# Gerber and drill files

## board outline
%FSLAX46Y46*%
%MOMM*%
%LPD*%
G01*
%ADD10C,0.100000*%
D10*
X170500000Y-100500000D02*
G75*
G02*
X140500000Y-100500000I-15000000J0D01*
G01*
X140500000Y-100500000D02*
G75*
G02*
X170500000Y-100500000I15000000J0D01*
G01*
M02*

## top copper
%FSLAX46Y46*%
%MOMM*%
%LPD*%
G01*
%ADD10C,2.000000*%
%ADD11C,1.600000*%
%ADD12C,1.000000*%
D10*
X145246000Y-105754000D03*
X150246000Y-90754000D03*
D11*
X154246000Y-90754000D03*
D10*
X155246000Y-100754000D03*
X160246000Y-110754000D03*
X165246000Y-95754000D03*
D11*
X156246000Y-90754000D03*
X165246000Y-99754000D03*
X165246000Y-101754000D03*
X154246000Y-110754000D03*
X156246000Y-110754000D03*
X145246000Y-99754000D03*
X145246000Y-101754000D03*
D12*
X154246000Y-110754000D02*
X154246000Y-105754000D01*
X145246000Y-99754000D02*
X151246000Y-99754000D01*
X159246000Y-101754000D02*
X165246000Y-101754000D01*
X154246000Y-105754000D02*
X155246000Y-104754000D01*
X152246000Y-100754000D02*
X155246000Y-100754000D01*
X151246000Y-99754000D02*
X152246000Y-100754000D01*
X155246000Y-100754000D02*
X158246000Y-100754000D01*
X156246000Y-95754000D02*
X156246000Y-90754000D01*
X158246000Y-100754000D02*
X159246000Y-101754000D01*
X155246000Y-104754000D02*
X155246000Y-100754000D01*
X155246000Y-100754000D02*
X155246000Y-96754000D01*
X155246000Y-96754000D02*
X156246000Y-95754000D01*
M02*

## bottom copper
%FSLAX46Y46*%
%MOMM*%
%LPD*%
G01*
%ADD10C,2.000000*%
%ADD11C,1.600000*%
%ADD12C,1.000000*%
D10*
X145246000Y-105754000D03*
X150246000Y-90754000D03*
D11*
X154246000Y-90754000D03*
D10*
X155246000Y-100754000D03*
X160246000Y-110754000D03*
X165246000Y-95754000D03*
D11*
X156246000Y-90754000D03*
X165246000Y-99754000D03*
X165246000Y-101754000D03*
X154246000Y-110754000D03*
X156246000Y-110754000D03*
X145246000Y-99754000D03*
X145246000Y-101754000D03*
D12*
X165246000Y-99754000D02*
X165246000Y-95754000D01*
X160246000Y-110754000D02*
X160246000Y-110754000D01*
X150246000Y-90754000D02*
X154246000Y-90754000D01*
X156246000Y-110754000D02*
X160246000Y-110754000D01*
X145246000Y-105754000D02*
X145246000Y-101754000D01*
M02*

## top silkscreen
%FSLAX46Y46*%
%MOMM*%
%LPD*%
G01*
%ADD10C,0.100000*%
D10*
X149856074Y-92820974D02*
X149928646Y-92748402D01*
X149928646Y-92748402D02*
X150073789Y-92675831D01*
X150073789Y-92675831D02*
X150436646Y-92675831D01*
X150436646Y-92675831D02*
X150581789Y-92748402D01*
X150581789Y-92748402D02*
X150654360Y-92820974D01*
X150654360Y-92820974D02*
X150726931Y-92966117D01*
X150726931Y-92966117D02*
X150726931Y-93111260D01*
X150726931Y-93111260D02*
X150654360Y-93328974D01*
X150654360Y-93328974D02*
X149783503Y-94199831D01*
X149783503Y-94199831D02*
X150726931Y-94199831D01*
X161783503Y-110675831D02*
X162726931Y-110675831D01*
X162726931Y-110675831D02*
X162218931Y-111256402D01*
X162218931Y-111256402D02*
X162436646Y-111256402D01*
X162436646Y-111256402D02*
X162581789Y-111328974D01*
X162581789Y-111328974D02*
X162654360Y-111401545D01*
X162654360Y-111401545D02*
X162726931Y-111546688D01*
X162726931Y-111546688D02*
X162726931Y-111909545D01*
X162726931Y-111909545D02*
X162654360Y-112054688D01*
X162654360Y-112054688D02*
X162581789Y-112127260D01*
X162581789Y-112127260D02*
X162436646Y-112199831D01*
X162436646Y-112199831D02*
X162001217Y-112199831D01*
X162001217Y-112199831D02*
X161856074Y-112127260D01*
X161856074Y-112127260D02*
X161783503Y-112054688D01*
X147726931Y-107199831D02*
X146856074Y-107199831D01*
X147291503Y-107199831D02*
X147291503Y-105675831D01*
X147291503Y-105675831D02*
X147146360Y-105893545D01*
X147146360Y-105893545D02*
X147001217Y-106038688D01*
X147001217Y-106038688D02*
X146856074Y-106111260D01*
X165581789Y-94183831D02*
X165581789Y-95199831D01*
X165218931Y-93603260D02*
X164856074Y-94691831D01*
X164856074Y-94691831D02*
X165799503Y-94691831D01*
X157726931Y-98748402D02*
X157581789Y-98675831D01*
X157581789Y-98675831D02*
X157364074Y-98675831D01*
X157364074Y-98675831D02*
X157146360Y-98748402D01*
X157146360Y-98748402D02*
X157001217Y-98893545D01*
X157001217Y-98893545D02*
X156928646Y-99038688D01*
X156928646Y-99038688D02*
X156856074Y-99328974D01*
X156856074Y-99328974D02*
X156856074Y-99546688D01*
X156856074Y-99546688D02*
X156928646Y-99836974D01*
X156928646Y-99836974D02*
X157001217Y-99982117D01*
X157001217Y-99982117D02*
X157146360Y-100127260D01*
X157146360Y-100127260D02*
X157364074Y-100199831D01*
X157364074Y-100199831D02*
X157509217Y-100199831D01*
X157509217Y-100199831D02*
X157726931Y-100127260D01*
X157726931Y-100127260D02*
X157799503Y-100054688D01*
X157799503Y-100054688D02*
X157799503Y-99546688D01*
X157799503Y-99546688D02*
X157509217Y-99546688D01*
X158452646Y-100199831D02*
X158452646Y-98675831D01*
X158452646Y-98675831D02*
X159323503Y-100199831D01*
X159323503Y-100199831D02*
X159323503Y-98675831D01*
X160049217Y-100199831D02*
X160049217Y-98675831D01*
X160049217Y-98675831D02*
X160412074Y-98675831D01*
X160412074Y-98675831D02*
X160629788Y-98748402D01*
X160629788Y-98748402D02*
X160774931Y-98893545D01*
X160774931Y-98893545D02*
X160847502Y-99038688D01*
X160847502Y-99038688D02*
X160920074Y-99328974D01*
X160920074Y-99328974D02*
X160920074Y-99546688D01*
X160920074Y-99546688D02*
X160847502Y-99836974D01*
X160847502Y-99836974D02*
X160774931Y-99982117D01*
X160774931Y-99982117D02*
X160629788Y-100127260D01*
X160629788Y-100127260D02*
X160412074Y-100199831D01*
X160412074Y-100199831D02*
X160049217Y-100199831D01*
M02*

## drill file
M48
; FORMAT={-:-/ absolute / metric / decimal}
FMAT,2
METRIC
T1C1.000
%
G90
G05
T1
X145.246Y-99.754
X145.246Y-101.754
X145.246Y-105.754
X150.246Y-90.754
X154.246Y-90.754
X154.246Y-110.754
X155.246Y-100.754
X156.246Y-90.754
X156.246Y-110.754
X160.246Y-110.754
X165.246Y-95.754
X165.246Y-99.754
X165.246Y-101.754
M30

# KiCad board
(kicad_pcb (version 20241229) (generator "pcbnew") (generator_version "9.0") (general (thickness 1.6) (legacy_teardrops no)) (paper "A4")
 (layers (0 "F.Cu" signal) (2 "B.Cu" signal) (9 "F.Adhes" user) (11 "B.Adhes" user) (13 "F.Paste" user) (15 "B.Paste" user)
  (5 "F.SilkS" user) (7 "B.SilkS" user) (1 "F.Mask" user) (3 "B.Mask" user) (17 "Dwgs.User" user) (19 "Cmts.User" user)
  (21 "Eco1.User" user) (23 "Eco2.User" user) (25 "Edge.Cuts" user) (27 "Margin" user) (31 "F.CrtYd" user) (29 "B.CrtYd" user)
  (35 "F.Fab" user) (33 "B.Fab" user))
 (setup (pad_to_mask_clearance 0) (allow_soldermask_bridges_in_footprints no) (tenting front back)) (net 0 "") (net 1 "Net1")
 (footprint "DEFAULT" (layer "F.Cu") (at 61.246 195.754)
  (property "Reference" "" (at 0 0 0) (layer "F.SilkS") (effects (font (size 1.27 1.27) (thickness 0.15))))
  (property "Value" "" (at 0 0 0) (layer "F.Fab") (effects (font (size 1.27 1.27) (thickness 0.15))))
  (pad "173" thru_hole circle (at 84 -90) (size 2 2) (drill 1) (layers "*.Cu") (remove_unused_layers no))
  (pad "173" thru_hole circle (at 89 -105) (size 2 2) (drill 1) (layers "*.Cu") (remove_unused_layers no))
  (pad "173" thru_hole circle (at 93 -105) (size 1.6 1.6) (drill 1) (layers "*.Cu") (remove_unused_layers no))
  (pad "173" thru_hole circle (at 94 -95) (size 2 2) (drill 1) (layers "*.Cu") (remove_unused_layers no))
  (pad "173" thru_hole circle (at 99 -85) (size 2 2) (drill 1) (layers "*.Cu") (remove_unused_layers no))
  (pad "173" thru_hole circle (at 104 -100) (size 2 2) (drill 1) (layers "*.Cu") (remove_unused_layers no))
  (pad "174" thru_hole circle (at 95 -105) (size 1.6 1.6) (drill 1) (layers "*.Cu") (remove_unused_layers no))
  (pad "175" thru_hole circle (at 104 -96) (size 1.6 1.6) (drill 1) (layers "*.Cu") (remove_unused_layers no))
  (pad "176" thru_hole circle (at 104 -94) (size 1.6 1.6) (drill 1) (layers "*.Cu") (remove_unused_layers no))
  (pad "177" thru_hole circle (at 93 -85) (size 1.6 1.6) (drill 1) (layers "*.Cu") (remove_unused_layers no))
  (pad "178" thru_hole circle (at 95 -85) (size 1.6 1.6) (drill 1) (layers "*.Cu") (remove_unused_layers no))
  (pad "179" thru_hole circle (at 84 -96) (size 1.6 1.6) (drill 1) (layers "*.Cu") (remove_unused_layers no))
  (pad "180" thru_hole circle (at 84 -94) (size 1.6 1.6) (drill 1) (layers "*.Cu") (remove_unused_layers no)))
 (gr_circle (center 155.5 100.5) (end 170.5 100.5) (stroke (width 0.1) (type solid)) (fill no) (layer "Edge.Cuts"))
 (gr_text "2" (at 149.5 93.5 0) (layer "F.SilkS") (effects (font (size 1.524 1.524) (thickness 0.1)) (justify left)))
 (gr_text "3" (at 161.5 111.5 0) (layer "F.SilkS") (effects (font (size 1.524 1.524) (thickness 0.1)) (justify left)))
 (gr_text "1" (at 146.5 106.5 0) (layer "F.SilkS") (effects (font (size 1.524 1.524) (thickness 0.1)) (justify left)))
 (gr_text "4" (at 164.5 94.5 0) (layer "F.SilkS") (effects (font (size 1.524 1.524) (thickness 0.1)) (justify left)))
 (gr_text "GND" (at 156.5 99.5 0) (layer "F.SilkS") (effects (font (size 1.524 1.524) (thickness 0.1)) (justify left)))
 (segment (start 154.246 110.754) (end 154.246 105.754) (width 1) (layer "F.Cu") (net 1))
 (segment (start 145.246 99.754) (end 151.246 99.754) (width 1) (layer "F.Cu") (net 1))
 (segment (start 159.246 101.754) (end 165.246 101.754) (width 1) (layer "F.Cu") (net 1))
 (segment (start 154.246 105.754) (end 155.246 104.754) (width 1) (layer "F.Cu") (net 1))
 (segment (start 152.246 100.754) (end 155.246 100.754) (width 1) (layer "F.Cu") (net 1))
 (segment (start 151.246 99.754) (end 152.246 100.754) (width 1) (layer "F.Cu") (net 1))
 (segment (start 155.246 100.754) (end 158.246 100.754) (width 1) (layer "F.Cu") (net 1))
 (segment (start 156.246 95.754) (end 156.246 90.754) (width 1) (layer "F.Cu") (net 1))
 (segment (start 158.246 100.754) (end 159.246 101.754) (width 1) (layer "F.Cu") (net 1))
 (segment (start 155.246 104.754) (end 155.246 100.754) (width 1) (layer "F.Cu") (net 1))
 (segment (start 155.246 100.754) (end 155.246 96.754) (width 1) (layer "F.Cu") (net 1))
 (segment (start 155.246 96.754) (end 156.246 95.754) (width 1) (layer "F.Cu") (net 1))
 (segment (start 165.246 99.754) (end 165.246 95.754) (width 1) (layer "B.Cu") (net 1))
 (segment (start 160.246 110.754) (end 160.246 110.754) (width 1) (layer "B.Cu") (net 1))
 (segment (start 150.246 90.754) (end 154.246 90.754) (width 1) (layer "B.Cu") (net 1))
 (segment (start 156.246 110.754) (end 160.246 110.754) (width 1) (layer "B.Cu") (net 1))
 (segment (start 145.246 105.754) (end 145.246 101.754) (width 1) (layer "B.Cu") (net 1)))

